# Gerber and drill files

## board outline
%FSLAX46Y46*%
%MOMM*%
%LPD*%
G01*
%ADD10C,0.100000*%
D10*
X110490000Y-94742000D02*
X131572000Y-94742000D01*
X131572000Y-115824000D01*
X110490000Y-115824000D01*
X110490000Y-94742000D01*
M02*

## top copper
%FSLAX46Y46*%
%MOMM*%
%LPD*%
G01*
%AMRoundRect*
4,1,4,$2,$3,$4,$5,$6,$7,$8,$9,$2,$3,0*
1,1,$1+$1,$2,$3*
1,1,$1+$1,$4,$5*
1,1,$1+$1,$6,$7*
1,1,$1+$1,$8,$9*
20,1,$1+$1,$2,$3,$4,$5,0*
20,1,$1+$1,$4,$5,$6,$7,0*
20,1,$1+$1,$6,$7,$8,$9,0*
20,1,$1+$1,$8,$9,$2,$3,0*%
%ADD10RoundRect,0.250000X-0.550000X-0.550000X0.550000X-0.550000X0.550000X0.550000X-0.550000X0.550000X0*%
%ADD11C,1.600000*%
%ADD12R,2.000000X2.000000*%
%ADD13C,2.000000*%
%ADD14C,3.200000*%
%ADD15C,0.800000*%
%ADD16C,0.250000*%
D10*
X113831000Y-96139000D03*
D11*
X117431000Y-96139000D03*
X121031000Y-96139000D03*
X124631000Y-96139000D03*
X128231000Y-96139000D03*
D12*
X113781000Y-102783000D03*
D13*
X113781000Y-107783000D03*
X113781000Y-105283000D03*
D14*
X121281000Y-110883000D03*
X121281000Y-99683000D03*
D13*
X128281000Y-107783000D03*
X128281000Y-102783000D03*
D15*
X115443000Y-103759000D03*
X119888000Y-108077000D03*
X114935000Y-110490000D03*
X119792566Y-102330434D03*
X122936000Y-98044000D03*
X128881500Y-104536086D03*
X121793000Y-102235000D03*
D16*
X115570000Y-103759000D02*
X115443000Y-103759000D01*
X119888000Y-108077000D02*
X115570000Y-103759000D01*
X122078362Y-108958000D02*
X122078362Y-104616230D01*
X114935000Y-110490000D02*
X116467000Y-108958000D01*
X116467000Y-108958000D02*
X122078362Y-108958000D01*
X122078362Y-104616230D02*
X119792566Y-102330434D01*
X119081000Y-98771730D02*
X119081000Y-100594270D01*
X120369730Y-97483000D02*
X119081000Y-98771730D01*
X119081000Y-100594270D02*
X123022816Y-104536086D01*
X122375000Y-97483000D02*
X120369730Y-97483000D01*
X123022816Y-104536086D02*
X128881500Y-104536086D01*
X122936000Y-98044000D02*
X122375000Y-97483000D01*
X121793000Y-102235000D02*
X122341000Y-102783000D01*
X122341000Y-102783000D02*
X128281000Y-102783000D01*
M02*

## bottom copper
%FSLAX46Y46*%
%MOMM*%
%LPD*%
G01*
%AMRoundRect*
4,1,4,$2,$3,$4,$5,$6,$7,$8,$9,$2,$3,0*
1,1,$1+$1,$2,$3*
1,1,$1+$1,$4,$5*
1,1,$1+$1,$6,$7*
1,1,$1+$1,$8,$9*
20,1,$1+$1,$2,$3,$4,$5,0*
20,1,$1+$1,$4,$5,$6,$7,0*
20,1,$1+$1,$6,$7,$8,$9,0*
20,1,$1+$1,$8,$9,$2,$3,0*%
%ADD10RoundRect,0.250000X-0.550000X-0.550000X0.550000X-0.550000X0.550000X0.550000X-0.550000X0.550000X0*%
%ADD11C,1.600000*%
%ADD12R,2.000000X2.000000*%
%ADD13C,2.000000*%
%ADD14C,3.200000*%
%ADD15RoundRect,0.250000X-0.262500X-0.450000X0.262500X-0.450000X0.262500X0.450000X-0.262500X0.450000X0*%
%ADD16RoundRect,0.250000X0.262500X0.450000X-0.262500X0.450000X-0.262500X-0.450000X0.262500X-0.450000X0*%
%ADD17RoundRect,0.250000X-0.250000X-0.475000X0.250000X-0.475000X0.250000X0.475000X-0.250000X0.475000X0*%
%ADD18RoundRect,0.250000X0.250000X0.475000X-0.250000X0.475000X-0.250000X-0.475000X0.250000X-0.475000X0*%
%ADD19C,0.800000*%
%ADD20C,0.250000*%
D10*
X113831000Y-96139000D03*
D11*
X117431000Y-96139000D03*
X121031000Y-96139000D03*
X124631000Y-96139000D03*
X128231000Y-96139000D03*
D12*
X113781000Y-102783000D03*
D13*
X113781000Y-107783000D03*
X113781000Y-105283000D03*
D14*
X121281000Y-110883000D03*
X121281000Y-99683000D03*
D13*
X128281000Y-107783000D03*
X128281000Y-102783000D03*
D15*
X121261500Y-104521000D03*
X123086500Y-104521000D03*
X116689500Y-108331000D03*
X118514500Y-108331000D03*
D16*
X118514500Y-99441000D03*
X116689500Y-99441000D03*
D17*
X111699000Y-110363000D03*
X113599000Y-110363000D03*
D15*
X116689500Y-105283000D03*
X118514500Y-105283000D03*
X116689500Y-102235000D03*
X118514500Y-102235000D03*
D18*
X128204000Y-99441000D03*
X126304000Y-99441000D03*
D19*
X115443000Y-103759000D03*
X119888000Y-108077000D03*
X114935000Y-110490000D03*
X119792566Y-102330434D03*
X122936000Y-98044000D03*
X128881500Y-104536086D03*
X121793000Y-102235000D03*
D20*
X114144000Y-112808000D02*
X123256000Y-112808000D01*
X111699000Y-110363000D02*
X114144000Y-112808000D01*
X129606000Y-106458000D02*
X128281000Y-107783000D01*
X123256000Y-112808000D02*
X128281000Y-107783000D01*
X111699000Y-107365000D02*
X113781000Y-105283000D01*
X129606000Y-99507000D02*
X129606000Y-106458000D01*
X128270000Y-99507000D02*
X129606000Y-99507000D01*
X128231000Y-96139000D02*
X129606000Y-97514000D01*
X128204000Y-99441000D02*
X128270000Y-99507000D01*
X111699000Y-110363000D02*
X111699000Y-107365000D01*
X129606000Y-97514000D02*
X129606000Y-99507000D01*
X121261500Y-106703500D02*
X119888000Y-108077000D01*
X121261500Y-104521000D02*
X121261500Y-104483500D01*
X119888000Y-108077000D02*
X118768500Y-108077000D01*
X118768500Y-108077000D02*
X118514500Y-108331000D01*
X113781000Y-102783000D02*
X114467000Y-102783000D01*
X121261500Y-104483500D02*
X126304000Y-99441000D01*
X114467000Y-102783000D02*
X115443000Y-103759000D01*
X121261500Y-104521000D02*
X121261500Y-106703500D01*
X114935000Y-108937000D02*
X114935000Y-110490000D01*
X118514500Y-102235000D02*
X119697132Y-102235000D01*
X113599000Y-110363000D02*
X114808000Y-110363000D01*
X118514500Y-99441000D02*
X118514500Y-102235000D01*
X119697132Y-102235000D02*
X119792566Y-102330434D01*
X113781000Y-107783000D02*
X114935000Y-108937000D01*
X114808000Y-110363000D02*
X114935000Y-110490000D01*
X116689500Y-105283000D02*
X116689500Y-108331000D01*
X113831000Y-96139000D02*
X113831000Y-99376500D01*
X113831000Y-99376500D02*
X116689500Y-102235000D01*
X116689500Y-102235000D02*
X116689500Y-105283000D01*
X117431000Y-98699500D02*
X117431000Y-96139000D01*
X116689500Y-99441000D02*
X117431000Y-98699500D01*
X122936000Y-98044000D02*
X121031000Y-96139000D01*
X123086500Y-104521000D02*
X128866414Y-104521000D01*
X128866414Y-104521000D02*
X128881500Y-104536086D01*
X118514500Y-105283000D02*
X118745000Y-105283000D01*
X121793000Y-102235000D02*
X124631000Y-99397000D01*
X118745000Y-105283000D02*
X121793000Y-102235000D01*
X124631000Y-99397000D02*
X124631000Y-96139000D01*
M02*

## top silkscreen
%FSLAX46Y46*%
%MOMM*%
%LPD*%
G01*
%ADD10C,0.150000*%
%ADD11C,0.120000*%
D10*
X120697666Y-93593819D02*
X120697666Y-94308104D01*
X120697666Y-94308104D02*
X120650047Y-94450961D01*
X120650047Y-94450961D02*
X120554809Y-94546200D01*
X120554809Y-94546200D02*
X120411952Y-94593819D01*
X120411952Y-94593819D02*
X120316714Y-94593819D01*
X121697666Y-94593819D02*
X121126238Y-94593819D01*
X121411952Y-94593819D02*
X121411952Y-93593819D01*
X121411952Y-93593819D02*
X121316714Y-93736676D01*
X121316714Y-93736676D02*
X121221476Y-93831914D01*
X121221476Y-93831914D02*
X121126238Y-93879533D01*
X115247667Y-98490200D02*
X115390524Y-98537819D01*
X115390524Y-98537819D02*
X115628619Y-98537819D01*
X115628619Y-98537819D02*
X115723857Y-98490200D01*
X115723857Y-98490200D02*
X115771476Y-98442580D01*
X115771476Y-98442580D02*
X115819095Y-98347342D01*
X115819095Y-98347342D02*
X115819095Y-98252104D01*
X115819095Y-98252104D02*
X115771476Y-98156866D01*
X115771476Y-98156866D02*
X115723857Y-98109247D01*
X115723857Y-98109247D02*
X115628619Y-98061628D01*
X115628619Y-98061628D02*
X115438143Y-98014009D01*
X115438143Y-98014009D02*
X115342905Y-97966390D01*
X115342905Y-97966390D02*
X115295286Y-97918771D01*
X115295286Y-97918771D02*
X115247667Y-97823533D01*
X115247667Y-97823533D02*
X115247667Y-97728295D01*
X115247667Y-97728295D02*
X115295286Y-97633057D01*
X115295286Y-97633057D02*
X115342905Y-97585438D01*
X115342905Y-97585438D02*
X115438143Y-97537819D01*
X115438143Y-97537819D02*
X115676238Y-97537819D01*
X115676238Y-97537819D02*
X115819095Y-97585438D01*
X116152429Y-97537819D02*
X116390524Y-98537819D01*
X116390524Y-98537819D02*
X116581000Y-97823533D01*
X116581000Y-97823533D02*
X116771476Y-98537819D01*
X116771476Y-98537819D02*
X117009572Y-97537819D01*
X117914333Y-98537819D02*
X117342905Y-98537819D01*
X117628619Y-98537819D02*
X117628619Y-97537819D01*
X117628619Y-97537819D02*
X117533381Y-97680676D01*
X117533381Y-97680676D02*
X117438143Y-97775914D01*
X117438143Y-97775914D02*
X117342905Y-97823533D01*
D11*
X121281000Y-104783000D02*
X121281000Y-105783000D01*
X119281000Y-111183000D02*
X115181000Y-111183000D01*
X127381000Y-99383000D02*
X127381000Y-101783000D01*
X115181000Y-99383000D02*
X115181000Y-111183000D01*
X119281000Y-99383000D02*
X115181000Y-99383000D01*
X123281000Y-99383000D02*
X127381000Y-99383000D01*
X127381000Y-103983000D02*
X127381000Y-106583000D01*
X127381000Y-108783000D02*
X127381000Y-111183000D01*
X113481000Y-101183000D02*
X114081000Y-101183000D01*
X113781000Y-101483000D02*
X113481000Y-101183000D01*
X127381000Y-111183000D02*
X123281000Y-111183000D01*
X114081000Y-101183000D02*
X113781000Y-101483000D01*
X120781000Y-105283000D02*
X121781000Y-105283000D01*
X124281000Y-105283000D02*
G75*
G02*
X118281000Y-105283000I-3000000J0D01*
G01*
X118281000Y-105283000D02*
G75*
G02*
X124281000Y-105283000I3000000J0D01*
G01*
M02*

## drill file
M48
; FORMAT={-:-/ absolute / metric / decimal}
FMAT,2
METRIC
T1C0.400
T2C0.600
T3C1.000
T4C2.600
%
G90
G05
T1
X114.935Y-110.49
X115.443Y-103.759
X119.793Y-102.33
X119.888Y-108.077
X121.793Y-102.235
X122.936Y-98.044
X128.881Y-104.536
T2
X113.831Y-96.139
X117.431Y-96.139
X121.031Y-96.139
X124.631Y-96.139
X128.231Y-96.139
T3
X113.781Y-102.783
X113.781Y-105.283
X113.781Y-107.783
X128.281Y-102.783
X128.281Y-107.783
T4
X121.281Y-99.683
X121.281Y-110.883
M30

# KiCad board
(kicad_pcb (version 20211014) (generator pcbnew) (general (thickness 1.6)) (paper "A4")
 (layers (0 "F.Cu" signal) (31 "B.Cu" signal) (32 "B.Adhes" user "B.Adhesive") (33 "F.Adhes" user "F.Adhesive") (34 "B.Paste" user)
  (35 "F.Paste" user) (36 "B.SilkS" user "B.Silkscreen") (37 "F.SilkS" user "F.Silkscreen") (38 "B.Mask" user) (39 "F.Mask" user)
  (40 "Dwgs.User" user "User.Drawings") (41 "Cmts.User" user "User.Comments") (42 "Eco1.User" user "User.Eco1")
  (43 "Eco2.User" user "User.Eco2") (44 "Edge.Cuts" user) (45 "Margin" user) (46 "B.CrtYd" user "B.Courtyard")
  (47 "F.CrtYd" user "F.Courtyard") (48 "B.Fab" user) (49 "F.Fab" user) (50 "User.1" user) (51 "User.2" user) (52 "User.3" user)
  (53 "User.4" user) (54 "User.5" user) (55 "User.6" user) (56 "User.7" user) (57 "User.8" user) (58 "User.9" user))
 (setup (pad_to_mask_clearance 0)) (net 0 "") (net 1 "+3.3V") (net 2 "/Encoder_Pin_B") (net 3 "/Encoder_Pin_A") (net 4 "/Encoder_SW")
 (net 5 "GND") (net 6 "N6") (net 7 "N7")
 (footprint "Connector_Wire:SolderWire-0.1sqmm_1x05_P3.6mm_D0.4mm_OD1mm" (layer "F.Cu") (at 113.831 96.139)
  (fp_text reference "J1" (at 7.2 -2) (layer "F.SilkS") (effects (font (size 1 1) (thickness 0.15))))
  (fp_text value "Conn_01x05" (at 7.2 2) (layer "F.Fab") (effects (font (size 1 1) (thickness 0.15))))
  (pad "1" thru_hole roundrect (at 0 0) (size 1.6 1.6) (drill 0.6) (layers *.Cu *.Mask) (roundrect_rratio 0.15625) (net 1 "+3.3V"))
  (pad "2" thru_hole circle (at 3.6 0) (size 1.6 1.6) (drill 0.6) (layers *.Cu *.Mask) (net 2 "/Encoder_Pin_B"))
  (pad "3" thru_hole circle (at 7.2 0) (size 1.6 1.6) (drill 0.6) (layers *.Cu *.Mask) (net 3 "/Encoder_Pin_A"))
  (pad "4" thru_hole circle (at 10.8 0) (size 1.6 1.6) (drill 0.6) (layers *.Cu *.Mask) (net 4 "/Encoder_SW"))
  (pad "5" thru_hole circle (at 14.4 0) (size 1.6 1.6) (drill 0.6) (layers *.Cu *.Mask) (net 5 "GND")))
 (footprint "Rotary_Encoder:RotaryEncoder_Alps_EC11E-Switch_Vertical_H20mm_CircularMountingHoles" (layer "F.Cu") (at 113.781 102.783)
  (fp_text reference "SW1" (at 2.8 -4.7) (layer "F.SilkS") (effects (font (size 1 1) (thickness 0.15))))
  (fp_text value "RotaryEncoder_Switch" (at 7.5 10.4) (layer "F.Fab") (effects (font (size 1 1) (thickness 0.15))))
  (fp_line (start 7.5 2) (end 7.5 3) (layer "F.SilkS") (width 0.12))
  (fp_line (start 5.5 8.4) (end 1.4 8.4) (layer "F.SilkS") (width 0.12))
  (fp_line (start 13.6 -3.4) (end 13.6 -1) (layer "F.SilkS") (width 0.12))
  (fp_line (start 1.4 -3.4) (end 1.4 8.4) (layer "F.SilkS") (width 0.12))
  (fp_line (start 5.5 -3.4) (end 1.4 -3.4) (layer "F.SilkS") (width 0.12))
  (fp_line (start 9.5 -3.4) (end 13.6 -3.4) (layer "F.SilkS") (width 0.12))
  (fp_line (start 13.6 1.2) (end 13.6 3.8) (layer "F.SilkS") (width 0.12))
  (fp_line (start 13.6 6) (end 13.6 8.4) (layer "F.SilkS") (width 0.12))
  (fp_line (start -0.3 -1.6) (end 0.3 -1.6) (layer "F.SilkS") (width 0.12))
  (fp_line (start 0 -1.3) (end -0.3 -1.6) (layer "F.SilkS") (width 0.12))
  (fp_line (start 13.6 8.4) (end 9.5 8.4) (layer "F.SilkS") (width 0.12))
  (fp_line (start 0.3 -1.6) (end 0 -1.3) (layer "F.SilkS") (width 0.12))
  (fp_line (start 7 2.5) (end 8 2.5) (layer "F.SilkS") (width 0.12))
  (fp_circle (center 7.5 2.5) (end 10.5 2.5) (layer "F.SilkS") (width 0.12) (fill none))
  (pad "A" thru_hole rect (at 0 0) (size 2 2) (drill 1) (layers *.Cu *.Mask) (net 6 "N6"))
  (pad "B" thru_hole circle (at 0 5) (size 2 2) (drill 1) (layers *.Cu *.Mask) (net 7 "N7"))
  (pad "C" thru_hole circle (at 0 2.5) (size 2 2) (drill 1) (layers *.Cu *.Mask) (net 5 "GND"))
  (pad "MP" thru_hole circle (at 7.5 8.1) (size 3.2 3.2) (drill 2.6) (layers *.Cu *.Mask))
  (pad "MP" thru_hole circle (at 7.5 -3.1) (size 3.2 3.2) (drill 2.6) (layers *.Cu *.Mask))
  (pad "S1" thru_hole circle (at 14.5 5) (size 2 2) (drill 1) (layers *.Cu *.Mask) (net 5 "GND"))
  (pad "S2" thru_hole circle (at 14.5 0) (size 2 2) (drill 1) (layers *.Cu *.Mask) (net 4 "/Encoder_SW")))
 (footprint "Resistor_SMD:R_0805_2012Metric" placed (layer "B.Cu") (at 122.174 104.521)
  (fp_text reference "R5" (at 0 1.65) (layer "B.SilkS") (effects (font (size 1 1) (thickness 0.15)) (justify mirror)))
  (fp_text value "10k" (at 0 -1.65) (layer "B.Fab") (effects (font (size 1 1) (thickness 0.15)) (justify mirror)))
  (pad "1" smd roundrect (at -0.9125 0) (size 1.025 1.4) (layers "B.Cu" "B.Paste" "B.Mask") (roundrect_rratio 0.243902439) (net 6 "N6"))
  (pad "2" smd roundrect (at 0.9125 0) (size 1.025 1.4) (layers "B.Cu" "B.Paste" "B.Mask") (roundrect_rratio 0.243902439)
   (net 3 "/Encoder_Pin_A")))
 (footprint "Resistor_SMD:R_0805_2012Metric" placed (layer "B.Cu") (at 117.602 108.331)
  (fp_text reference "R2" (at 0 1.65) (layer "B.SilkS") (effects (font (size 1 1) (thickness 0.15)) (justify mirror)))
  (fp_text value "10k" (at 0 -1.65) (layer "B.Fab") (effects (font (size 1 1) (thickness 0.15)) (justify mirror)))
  (pad "1" smd roundrect (at -0.9125 0) (size 1.025 1.4) (layers "B.Cu" "B.Paste" "B.Mask") (roundrect_rratio 0.243902439) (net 1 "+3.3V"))
  (pad "2" smd roundrect (at 0.9125 0) (size 1.025 1.4) (layers "B.Cu" "B.Paste" "B.Mask") (roundrect_rratio 0.243902439) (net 6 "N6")))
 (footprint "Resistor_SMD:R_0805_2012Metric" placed (layer "B.Cu") (at 117.602 99.441 180)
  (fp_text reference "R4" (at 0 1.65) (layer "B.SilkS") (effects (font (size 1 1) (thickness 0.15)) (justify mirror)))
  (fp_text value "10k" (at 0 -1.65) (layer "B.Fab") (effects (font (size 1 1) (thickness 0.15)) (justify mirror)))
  (pad "1" smd roundrect (at -0.9125 0 180) (size 1.025 1.4) (layers "B.Cu" "B.Paste" "B.Mask") (roundrect_rratio 0.243902439) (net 7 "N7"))
  (pad "2" smd roundrect (at 0.9125 0 180) (size 1.025 1.4) (layers "B.Cu" "B.Paste" "B.Mask") (roundrect_rratio 0.243902439)
   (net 2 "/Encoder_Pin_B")))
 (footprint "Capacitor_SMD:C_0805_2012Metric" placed (layer "B.Cu") (at 112.649 110.363)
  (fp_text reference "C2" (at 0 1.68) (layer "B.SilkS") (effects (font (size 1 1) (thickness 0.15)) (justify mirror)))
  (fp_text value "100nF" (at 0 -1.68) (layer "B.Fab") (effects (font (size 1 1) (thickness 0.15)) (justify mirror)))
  (pad "1" smd roundrect (at -0.95 0) (size 1 1.45) (layers "B.Cu" "B.Paste" "B.Mask") (roundrect_rratio 0.25) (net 5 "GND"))
  (pad "2" smd roundrect (at 0.95 0) (size 1 1.45) (layers "B.Cu" "B.Paste" "B.Mask") (roundrect_rratio 0.25) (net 7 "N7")))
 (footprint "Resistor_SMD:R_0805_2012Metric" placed (layer "B.Cu") (at 117.602 105.283)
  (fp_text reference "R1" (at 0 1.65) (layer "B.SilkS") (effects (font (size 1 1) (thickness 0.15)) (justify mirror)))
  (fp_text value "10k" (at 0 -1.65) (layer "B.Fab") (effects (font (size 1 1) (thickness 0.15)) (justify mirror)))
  (pad "1" smd roundrect (at -0.9125 0) (size 1.025 1.4) (layers "B.Cu" "B.Paste" "B.Mask") (roundrect_rratio 0.243902439) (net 1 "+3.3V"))
  (pad "2" smd roundrect (at 0.9125 0) (size 1.025 1.4) (layers "B.Cu" "B.Paste" "B.Mask") (roundrect_rratio 0.243902439)
   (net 4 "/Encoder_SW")))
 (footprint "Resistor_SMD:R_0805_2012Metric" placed (layer "B.Cu") (at 117.602 102.235)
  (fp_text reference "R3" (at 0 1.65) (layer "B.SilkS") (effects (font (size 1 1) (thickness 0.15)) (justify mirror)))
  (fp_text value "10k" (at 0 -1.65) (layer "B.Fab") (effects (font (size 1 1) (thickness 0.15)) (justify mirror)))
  (pad "1" smd roundrect (at -0.9125 0) (size 1.025 1.4) (layers "B.Cu" "B.Paste" "B.Mask") (roundrect_rratio 0.243902439) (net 1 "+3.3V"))
  (pad "2" smd roundrect (at 0.9125 0) (size 1.025 1.4) (layers "B.Cu" "B.Paste" "B.Mask") (roundrect_rratio 0.243902439) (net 7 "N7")))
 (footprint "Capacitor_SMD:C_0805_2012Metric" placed (layer "B.Cu") (at 127.254 99.441 180)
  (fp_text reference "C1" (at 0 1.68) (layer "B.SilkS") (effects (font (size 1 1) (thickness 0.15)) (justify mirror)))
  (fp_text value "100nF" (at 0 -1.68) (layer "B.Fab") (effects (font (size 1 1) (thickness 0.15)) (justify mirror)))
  (pad "1" smd roundrect (at -0.95 0 180) (size 1 1.45) (layers "B.Cu" "B.Paste" "B.Mask") (roundrect_rratio 0.25) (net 5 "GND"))
  (pad "2" smd roundrect (at 0.95 0 180) (size 1 1.45) (layers "B.Cu" "B.Paste" "B.Mask") (roundrect_rratio 0.25) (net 6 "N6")))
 (gr_rect (start 110.49 94.742) (end 131.572 115.824) (layer "Edge.Cuts") (width 0.1) (fill none))
 (segment (start 114.144 112.808) (end 123.256 112.808) (width 0.25) (layer "B.Cu") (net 5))
 (segment (start 111.699 110.363) (end 114.144 112.808) (width 0.25) (layer "B.Cu") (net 5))
 (segment (start 129.606 106.458) (end 128.281 107.783) (width 0.25) (layer "B.Cu") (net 5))
 (segment (start 123.256 112.808) (end 128.281 107.783) (width 0.25) (layer "B.Cu") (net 5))
 (segment (start 111.699 107.365) (end 113.781 105.283) (width 0.25) (layer "B.Cu") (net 5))
 (segment (start 129.606 99.507) (end 129.606 106.458) (width 0.25) (layer "B.Cu") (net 5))
 (segment (start 128.27 99.507) (end 129.606 99.507) (width 0.25) (layer "B.Cu") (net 5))
 (segment (start 128.231 96.139) (end 129.606 97.514) (width 0.25) (layer "B.Cu") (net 5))
 (segment (start 128.204 99.441) (end 128.27 99.507) (width 0.25) (layer "B.Cu") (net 5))
 (segment (start 111.699 110.363) (end 111.699 107.365) (width 0.25) (layer "B.Cu") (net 5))
 (segment (start 129.606 97.514) (end 129.606 99.507) (width 0.25) (layer "B.Cu") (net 5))
 (segment (start 115.57 103.759) (end 115.443 103.759) (width 0.25) (layer "F.Cu") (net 6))
 (segment (start 119.888 108.077) (end 115.57 103.759) (width 0.25) (layer "F.Cu") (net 6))
 (via (at 115.443 103.759) (size 0.8) (drill 0.4) (layers "F.Cu" "B.Cu") (free) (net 6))
 (via (at 119.888 108.077) (size 0.8) (drill 0.4) (layers "F.Cu" "B.Cu") (free) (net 6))
 (segment (start 121.2615 106.7035) (end 119.888 108.077) (width 0.25) (layer "B.Cu") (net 6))
 (segment (start 121.2615 104.521) (end 121.2615 104.4835) (width 0.25) (layer "B.Cu") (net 6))
 (segment (start 119.888 108.077) (end 118.7685 108.077) (width 0.25) (layer "B.Cu") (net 6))
 (segment (start 118.7685 108.077) (end 118.5145 108.331) (width 0.25) (layer "B.Cu") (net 6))
 (segment (start 113.781 102.783) (end 114.467 102.783) (width 0.25) (layer "B.Cu") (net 6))
 (segment (start 121.2615 104.4835) (end 126.304 99.441) (width 0.25) (layer "B.Cu") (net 6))
 (segment (start 114.467 102.783) (end 115.443 103.759) (width 0.25) (layer "B.Cu") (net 6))
 (segment (start 121.2615 104.521) (end 121.2615 106.7035) (width 0.25) (layer "B.Cu") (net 6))
 (segment (start 122.078362 108.958) (end 122.078362 104.61623) (width 0.25) (layer "F.Cu") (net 7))
 (segment (start 114.935 110.49) (end 116.467 108.958) (width 0.25) (layer "F.Cu") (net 7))
 (segment (start 116.467 108.958) (end 122.078362 108.958) (width 0.25) (layer "F.Cu") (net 7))
 (segment (start 122.078362 104.61623) (end 119.792566 102.330434) (width 0.25) (layer "F.Cu") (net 7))
 (via (at 114.935 110.49) (size 0.8) (drill 0.4) (layers "F.Cu" "B.Cu") (free) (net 7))
 (via (at 119.792566 102.330434) (size 0.8) (drill 0.4) (layers "F.Cu" "B.Cu") (free) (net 7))
 (segment (start 114.935 108.937) (end 114.935 110.49) (width 0.25) (layer "B.Cu") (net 7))
 (segment (start 118.5145 102.235) (end 119.697132 102.235) (width 0.25) (layer "B.Cu") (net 7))
 (segment (start 113.599 110.363) (end 114.808 110.363) (width 0.25) (layer "B.Cu") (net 7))
 (segment (start 118.5145 99.441) (end 118.5145 102.235) (width 0.25) (layer "B.Cu") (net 7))
 (segment (start 119.697132 102.235) (end 119.792566 102.330434) (width 0.25) (layer "B.Cu") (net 7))
 (segment (start 113.781 107.783) (end 114.935 108.937) (width 0.25) (layer "B.Cu") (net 7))
 (segment (start 114.808 110.363) (end 114.935 110.49) (width 0.25) (layer "B.Cu") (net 7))
 (segment (start 116.6895 105.283) (end 116.6895 108.331) (width 0.25) (layer "B.Cu") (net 1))
 (segment (start 113.831 96.139) (end 113.831 99.3765) (width 0.25) (layer "B.Cu") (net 1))
 (segment (start 113.831 99.3765) (end 116.6895 102.235) (width 0.25) (layer "B.Cu") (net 1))
 (segment (start 116.6895 102.235) (end 116.6895 105.283) (width 0.25) (layer "B.Cu") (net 1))
 (segment (start 117.431 98.6995) (end 117.431 96.139) (width 0.25) (layer "B.Cu") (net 2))
 (segment (start 116.6895 99.441) (end 117.431 98.6995) (width 0.25) (layer "B.Cu") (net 2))
 (segment (start 119.081 98.77173) (end 119.081 100.59427) (width 0.25) (layer "F.Cu") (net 3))
 (segment (start 120.36973 97.483) (end 119.081 98.77173) (width 0.25) (layer "F.Cu") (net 3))
 (segment (start 119.081 100.59427) (end 123.022816 104.536086) (width 0.25) (layer "F.Cu") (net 3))
 (segment (start 122.375 97.483) (end 120.36973 97.483) (width 0.25) (layer "F.Cu") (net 3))
 (segment (start 123.022816 104.536086) (end 128.8815 104.536086) (width 0.25) (layer "F.Cu") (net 3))
 (segment (start 122.936 98.044) (end 122.375 97.483) (width 0.25) (layer "F.Cu") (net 3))
 (via (at 122.936 98.044) (size 0.8) (drill 0.4) (layers "F.Cu" "B.Cu") (free) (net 3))
 (via (at 128.8815 104.536086) (size 0.8) (drill 0.4) (layers "F.Cu" "B.Cu") (free) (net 3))
 (segment (start 122.936 98.044) (end 121.031 96.139) (width 0.25) (layer "B.Cu") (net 3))
 (segment (start 123.0865 104.521) (end 128.866414 104.521) (width 0.25) (layer "B.Cu") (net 3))
 (segment (start 128.866414 104.521) (end 128.8815 104.536086) (width 0.25) (layer "B.Cu") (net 3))
 (segment (start 121.793 102.235) (end 122.341 102.783) (width 0.25) (layer "F.Cu") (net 4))
 (segment (start 122.341 102.783) (end 128.281 102.783) (width 0.25) (layer "F.Cu") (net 4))
 (via (at 121.793 102.235) (size 0.8) (drill 0.4) (layers "F.Cu" "B.Cu") (free) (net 4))
 (segment (start 118.5145 105.283) (end 118.745 105.283) (width 0.25) (layer "B.Cu") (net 4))
 (segment (start 121.793 102.235) (end 124.631 99.397) (width 0.25) (layer "B.Cu") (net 4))
 (segment (start 118.745 105.283) (end 121.793 102.235) (width 0.25) (layer "B.Cu") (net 4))
 (segment (start 124.631 99.397) (end 124.631 96.139) (width 0.25) (layer "B.Cu") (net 4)))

